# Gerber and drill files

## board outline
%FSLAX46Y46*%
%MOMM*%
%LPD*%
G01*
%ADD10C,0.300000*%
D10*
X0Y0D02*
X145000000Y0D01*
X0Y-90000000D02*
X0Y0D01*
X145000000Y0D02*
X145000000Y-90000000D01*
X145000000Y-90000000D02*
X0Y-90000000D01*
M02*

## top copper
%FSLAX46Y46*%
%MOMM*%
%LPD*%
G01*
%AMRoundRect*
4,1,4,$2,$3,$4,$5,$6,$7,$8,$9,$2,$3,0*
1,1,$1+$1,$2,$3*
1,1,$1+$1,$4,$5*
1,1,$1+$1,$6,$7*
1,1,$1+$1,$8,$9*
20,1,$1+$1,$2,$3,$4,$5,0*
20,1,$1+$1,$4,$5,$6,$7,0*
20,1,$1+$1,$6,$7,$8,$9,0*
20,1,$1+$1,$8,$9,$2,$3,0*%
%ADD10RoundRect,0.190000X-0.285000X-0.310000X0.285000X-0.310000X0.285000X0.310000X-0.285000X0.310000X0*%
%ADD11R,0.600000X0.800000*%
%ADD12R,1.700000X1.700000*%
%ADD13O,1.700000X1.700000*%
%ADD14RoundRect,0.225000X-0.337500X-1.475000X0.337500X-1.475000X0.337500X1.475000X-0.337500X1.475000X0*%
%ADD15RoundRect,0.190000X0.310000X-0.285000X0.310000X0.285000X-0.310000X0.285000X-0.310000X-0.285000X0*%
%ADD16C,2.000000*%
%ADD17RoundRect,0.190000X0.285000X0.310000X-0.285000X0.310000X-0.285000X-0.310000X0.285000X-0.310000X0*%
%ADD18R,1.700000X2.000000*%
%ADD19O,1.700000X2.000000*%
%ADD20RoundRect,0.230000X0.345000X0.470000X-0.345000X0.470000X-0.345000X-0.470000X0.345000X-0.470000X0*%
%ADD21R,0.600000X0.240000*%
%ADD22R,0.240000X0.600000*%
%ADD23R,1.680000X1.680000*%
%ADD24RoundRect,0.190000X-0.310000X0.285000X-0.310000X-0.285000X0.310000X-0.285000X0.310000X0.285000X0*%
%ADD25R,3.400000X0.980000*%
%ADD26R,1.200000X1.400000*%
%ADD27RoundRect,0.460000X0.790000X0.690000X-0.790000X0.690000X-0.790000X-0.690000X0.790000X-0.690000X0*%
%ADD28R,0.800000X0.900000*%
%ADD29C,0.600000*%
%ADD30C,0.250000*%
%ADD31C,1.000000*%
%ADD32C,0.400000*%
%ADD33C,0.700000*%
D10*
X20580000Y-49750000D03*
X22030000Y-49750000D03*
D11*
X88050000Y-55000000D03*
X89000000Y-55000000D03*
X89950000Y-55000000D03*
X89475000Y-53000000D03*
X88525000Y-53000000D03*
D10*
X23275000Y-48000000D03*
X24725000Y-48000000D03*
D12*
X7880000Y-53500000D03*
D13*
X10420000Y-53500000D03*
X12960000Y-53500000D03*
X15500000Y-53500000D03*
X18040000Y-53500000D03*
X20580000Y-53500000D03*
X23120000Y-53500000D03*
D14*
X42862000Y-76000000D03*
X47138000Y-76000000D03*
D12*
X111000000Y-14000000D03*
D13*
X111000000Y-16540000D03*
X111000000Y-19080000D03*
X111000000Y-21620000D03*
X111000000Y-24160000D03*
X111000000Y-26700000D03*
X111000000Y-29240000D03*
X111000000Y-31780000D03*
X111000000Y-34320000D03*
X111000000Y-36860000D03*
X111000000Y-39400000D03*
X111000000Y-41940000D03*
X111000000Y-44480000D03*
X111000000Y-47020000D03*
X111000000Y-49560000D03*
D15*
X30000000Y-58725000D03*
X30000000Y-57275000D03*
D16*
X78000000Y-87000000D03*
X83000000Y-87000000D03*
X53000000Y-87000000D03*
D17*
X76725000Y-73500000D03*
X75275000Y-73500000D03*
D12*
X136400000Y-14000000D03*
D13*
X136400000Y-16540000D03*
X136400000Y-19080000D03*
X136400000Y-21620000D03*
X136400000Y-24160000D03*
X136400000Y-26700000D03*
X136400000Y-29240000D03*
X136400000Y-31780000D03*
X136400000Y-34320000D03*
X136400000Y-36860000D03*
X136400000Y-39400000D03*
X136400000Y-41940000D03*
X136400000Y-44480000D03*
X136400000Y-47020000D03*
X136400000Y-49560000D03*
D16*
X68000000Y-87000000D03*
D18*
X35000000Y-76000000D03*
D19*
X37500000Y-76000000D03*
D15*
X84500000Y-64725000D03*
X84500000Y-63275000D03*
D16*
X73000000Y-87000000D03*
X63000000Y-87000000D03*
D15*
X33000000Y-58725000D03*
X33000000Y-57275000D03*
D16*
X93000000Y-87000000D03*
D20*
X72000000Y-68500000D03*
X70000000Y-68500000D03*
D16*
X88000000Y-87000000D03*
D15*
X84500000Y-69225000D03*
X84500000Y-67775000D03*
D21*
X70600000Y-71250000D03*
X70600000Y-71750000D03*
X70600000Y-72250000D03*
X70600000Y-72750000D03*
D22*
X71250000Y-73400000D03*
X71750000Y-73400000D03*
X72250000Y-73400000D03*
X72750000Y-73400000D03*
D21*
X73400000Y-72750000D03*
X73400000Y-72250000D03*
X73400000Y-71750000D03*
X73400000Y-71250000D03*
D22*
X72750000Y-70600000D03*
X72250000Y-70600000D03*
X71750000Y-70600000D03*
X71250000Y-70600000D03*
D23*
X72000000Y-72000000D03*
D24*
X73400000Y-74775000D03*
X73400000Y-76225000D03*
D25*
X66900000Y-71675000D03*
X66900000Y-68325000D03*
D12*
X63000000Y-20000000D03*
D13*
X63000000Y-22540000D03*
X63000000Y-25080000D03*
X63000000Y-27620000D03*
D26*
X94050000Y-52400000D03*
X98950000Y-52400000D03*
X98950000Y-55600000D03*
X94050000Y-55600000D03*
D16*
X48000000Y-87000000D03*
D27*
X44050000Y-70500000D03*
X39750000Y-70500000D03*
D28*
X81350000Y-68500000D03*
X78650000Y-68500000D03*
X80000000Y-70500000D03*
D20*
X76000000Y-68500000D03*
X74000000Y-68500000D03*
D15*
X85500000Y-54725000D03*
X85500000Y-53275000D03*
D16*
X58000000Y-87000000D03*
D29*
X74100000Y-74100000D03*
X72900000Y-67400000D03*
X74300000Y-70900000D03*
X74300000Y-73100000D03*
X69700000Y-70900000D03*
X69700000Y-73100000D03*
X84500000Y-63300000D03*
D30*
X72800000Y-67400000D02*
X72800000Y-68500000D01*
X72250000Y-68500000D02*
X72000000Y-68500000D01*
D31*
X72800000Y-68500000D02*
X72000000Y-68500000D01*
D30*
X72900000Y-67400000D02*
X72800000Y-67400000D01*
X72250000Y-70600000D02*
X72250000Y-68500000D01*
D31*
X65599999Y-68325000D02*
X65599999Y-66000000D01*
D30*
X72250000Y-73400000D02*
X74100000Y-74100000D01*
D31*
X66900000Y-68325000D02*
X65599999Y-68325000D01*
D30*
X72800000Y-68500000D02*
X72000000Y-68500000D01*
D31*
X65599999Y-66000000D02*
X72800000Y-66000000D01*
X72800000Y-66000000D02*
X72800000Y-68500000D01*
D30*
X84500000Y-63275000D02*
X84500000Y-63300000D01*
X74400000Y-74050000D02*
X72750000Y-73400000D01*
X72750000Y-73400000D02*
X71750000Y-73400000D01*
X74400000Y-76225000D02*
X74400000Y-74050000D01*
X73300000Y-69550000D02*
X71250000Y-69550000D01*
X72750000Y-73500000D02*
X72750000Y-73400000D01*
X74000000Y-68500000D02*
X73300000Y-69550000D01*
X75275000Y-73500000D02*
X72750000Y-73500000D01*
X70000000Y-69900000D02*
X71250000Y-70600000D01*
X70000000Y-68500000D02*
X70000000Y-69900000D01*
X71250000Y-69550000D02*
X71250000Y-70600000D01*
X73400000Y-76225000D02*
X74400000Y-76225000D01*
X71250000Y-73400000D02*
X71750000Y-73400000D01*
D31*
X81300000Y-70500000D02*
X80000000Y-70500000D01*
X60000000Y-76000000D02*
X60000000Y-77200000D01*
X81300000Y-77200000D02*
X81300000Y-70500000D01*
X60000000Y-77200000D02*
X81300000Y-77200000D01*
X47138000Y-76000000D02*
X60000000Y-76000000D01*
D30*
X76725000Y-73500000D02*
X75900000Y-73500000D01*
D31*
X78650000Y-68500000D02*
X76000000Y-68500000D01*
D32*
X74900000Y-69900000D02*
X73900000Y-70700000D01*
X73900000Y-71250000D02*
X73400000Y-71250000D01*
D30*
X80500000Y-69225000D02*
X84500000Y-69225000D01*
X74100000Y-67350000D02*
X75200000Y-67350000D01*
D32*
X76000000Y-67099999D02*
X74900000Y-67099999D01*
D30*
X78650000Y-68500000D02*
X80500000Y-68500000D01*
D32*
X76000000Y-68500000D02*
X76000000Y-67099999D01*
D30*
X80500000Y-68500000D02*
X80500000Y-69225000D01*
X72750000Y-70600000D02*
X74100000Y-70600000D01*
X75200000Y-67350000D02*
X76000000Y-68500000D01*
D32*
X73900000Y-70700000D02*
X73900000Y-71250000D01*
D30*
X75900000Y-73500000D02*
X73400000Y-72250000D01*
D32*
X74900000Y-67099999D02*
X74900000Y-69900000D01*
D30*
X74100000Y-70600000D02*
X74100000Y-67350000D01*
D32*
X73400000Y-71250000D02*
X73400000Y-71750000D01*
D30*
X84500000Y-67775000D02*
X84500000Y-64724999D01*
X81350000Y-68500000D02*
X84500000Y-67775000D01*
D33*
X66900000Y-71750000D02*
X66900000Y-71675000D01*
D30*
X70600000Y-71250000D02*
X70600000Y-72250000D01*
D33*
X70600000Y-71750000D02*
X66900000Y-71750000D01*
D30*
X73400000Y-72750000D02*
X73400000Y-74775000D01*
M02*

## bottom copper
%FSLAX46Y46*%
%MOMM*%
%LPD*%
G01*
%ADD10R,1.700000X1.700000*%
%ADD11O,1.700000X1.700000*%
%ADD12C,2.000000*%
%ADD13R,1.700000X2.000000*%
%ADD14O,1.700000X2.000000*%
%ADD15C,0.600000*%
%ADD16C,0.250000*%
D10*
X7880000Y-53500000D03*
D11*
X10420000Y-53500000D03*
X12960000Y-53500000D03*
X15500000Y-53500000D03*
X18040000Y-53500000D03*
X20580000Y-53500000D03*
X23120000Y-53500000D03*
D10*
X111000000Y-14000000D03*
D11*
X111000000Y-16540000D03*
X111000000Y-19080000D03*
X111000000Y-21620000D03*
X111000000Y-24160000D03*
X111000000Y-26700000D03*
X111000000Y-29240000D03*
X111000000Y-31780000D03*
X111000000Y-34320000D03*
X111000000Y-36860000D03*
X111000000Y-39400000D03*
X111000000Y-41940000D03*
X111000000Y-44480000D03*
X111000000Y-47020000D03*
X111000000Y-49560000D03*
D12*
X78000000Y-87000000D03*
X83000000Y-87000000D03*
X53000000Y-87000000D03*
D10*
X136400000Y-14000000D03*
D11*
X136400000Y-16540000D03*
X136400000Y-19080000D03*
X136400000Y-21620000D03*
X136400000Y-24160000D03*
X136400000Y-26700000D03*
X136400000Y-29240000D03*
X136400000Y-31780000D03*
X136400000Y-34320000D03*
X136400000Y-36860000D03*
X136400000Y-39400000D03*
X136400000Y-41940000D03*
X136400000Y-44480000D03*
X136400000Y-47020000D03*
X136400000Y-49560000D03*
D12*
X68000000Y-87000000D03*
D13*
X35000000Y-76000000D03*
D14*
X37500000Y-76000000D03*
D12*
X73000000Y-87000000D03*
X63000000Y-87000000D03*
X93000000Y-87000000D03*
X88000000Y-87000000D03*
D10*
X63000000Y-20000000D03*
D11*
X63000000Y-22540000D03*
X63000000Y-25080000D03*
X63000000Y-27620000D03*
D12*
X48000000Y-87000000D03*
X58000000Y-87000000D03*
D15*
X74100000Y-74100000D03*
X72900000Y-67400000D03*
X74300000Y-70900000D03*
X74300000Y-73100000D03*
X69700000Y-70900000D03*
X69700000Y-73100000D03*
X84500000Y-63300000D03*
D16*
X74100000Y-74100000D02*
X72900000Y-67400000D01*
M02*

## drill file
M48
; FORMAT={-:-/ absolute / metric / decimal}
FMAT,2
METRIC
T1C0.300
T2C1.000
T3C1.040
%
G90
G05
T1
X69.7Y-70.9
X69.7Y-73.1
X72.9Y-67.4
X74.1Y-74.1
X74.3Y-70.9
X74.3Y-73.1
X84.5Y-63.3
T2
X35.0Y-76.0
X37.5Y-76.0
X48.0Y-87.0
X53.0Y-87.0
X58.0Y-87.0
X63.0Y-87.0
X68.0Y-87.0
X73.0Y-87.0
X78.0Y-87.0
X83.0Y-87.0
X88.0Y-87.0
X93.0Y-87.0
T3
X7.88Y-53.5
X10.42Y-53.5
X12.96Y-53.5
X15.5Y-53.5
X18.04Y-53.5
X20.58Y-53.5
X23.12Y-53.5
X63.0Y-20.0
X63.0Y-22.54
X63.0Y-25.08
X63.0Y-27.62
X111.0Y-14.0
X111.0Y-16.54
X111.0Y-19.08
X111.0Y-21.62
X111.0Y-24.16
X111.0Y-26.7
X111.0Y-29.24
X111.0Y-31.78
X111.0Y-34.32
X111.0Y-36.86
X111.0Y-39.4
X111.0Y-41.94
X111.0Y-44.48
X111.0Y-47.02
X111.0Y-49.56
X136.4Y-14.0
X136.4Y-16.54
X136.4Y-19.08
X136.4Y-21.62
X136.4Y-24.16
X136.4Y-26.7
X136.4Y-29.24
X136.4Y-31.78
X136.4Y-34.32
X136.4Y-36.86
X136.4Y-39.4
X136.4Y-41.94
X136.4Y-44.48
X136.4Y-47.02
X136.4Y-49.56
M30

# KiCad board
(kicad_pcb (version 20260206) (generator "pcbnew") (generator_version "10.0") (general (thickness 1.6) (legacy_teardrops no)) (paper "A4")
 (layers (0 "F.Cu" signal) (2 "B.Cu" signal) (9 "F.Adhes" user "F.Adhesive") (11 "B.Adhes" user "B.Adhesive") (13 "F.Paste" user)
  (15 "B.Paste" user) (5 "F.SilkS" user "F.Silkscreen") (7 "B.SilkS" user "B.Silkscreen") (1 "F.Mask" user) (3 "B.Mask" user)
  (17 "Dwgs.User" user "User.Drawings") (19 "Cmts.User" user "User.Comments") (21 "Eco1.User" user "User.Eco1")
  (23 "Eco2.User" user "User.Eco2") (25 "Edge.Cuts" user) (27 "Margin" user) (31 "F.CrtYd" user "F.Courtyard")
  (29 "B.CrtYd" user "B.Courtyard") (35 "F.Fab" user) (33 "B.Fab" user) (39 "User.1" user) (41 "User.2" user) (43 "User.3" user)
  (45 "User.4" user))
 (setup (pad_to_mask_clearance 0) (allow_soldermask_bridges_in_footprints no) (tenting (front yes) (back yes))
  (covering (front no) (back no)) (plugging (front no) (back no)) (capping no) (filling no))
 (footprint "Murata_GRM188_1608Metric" (layer "F.Cu") (at 21.305 49.75)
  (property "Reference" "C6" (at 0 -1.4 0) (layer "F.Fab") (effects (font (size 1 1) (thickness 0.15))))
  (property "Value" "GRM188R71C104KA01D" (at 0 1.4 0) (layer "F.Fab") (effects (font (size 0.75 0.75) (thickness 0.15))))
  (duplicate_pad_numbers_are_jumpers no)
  (pad "1" smd roundrect (at -0.725 0) (size 0.95 1) (layers "F.Cu" "F.Mask" "F.Paste") (roundrect_rratio 0.2) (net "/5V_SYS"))
  (pad "2" smd roundrect (at 0.725 0) (size 0.95 1) (layers "F.Cu" "F.Mask" "F.Paste") (roundrect_rratio 0.2) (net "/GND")))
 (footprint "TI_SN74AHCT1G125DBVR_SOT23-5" (layer "F.Cu") (at 89 54)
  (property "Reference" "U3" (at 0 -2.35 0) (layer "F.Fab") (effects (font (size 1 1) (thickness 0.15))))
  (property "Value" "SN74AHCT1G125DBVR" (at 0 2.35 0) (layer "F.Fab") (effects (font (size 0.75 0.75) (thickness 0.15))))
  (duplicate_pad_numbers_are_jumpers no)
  (pad "1" smd rect (at -0.95 1) (size 0.6 0.8) (layers "F.Cu" "F.Mask" "F.Paste") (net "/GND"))
  (pad "2" smd rect (at 0 1) (size 0.6 0.8) (layers "F.Cu" "F.Mask" "F.Paste") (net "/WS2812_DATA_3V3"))
  (pad "3" smd rect (at 0.95 1) (size 0.6 0.8) (layers "F.Cu" "F.Mask" "F.Paste") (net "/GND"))
  (pad "4" smd rect (at 0.475 -1) (size 0.6 0.8) (layers "F.Cu" "F.Mask" "F.Paste") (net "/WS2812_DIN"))
  (pad "5" smd rect (at -0.475 -1) (size 0.6 0.8) (layers "F.Cu" "F.Mask" "F.Paste") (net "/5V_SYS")))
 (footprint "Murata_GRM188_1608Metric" (layer "F.Cu") (at 24 48)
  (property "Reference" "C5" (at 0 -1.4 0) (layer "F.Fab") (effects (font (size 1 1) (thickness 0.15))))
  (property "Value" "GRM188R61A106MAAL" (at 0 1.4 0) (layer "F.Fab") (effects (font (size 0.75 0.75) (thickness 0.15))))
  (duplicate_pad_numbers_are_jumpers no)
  (pad "1" smd roundrect (at -0.725 0) (size 0.95 1) (layers "F.Cu" "F.Mask" "F.Paste") (roundrect_rratio 0.2) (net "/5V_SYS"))
  (pad "2" smd roundrect (at 0.725 0) (size 0.95 1) (layers "F.Cu" "F.Mask" "F.Paste") (roundrect_rratio 0.2) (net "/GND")))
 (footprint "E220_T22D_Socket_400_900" (layer "F.Cu") (at 5 52)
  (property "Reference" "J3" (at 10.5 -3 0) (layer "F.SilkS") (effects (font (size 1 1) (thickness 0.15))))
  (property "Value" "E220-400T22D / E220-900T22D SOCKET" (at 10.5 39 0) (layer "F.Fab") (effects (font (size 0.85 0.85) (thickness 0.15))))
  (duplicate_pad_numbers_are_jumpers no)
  (pad "1" thru_hole rect (at 2.88 1.5) (size 1.7 1.7) (drill 1.04) (layers "*.Cu" "*.Mask") (remove_unused_layers no) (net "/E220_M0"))
  (pad "2" thru_hole oval (at 5.42 1.5) (size 1.7 1.7) (drill 1.04) (layers "*.Cu" "*.Mask") (remove_unused_layers no) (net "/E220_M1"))
  (pad "3" thru_hole oval (at 7.96 1.5) (size 1.7 1.7) (drill 1.04) (layers "*.Cu" "*.Mask") (remove_unused_layers no) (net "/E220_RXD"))
  (pad "4" thru_hole oval (at 10.5 1.5) (size 1.7 1.7) (drill 1.04) (layers "*.Cu" "*.Mask") (remove_unused_layers no) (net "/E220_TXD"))
  (pad "5" thru_hole oval (at 13.04 1.5) (size 1.7 1.7) (drill 1.04) (layers "*.Cu" "*.Mask") (remove_unused_layers no) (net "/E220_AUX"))
  (pad "6" thru_hole oval (at 15.58 1.5) (size 1.7 1.7) (drill 1.04) (layers "*.Cu" "*.Mask") (remove_unused_layers no) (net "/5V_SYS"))
  (pad "7" thru_hole oval (at 18.12 1.5) (size 1.7 1.7) (drill 1.04) (layers "*.Cu" "*.Mask") (remove_unused_layers no) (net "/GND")))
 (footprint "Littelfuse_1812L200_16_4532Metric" (layer "F.Cu") (at 45 76)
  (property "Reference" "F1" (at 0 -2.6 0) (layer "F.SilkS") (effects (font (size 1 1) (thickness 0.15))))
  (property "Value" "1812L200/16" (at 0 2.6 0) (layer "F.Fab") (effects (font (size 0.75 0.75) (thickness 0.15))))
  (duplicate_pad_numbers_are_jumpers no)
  (pad "1" smd roundrect (at -2.138 0) (size 1.125 3.4) (layers "F.Cu" "F.Mask" "F.Paste") (roundrect_rratio 0.2) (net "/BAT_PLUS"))
  (pad "2" smd roundrect (at 2.138 0) (size 1.125 3.4) (layers "F.Cu" "F.Mask" "F.Paste") (roundrect_rratio 0.2) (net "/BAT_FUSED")))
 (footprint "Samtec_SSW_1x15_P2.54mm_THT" (layer "F.Cu") (at 111 14)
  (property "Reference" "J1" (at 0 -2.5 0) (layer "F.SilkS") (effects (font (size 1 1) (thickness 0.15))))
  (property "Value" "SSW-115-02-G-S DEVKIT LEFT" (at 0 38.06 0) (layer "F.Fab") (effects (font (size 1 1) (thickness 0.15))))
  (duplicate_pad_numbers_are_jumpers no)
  (pad "1" thru_hole rect (at 0 0) (size 1.7 1.7) (drill 1.04) (layers "*.Cu" "*.Mask") (remove_unused_layers no) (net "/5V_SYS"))
  (pad "2" thru_hole oval (at 0 2.54) (size 1.7 1.7) (drill 1.04) (layers "*.Cu" "*.Mask") (remove_unused_layers no) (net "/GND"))
  (pad "3" thru_hole oval (at 0 5.08) (size 1.7 1.7) (drill 1.04) (layers "*.Cu" "*.Mask") (remove_unused_layers no))
  (pad "4" thru_hole oval (at 0 7.62) (size 1.7 1.7) (drill 1.04) (layers "*.Cu" "*.Mask") (remove_unused_layers no))
  (pad "5" thru_hole oval (at 0 10.16) (size 1.7 1.7) (drill 1.04) (layers "*.Cu" "*.Mask") (remove_unused_layers no))
  (pad "6" thru_hole oval (at 0 12.7) (size 1.7 1.7) (drill 1.04) (layers "*.Cu" "*.Mask") (remove_unused_layers no) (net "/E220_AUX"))
  (pad "7" thru_hole oval (at 0 15.24) (size 1.7 1.7) (drill 1.04) (layers "*.Cu" "*.Mask") (remove_unused_layers no) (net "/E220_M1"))
  (pad "8" thru_hole oval (at 0 17.78) (size 1.7 1.7) (drill 1.04) (layers "*.Cu" "*.Mask") (remove_unused_layers no) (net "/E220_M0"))
  (pad "9" thru_hole oval (at 0 20.32) (size 1.7 1.7) (drill 1.04) (layers "*.Cu" "*.Mask") (remove_unused_layers no))
  (pad "10" thru_hole oval (at 0 22.86) (size 1.7 1.7) (drill 1.04) (layers "*.Cu" "*.Mask") (remove_unused_layers no))
  (pad "11" thru_hole oval (at 0 25.4) (size 1.7 1.7) (drill 1.04) (layers "*.Cu" "*.Mask") (remove_unused_layers no))
  (pad "12" thru_hole oval (at 0 27.94) (size 1.7 1.7) (drill 1.04) (layers "*.Cu" "*.Mask") (remove_unused_layers no))
  (pad "13" thru_hole oval (at 0 30.48) (size 1.7 1.7) (drill 1.04) (layers "*.Cu" "*.Mask") (remove_unused_layers no))
  (pad "14" thru_hole oval (at 0 33.02) (size 1.7 1.7) (drill 1.04) (layers "*.Cu" "*.Mask") (remove_unused_layers no))
  (pad "15" thru_hole oval (at 0 35.56) (size 1.7 1.7) (drill 1.04) (layers "*.Cu" "*.Mask") (remove_unused_layers no)))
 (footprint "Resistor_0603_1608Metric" (layer "F.Cu") (at 30 58 90)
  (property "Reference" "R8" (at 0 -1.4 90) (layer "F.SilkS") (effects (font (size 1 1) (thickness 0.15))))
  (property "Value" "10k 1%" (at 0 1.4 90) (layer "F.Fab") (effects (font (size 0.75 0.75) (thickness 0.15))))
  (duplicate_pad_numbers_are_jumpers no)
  (pad "1" smd roundrect (at -0.725 0 90) (size 0.95 1) (layers "F.Cu" "F.Mask" "F.Paste") (roundrect_rratio 0.2) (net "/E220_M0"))
  (pad "2" smd roundrect (at 0.725 0 90) (size 0.95 1) (layers "F.Cu" "F.Mask" "F.Paste") (roundrect_rratio 0.2) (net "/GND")))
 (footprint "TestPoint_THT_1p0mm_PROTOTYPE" (layer "F.Cu") (at 78 87)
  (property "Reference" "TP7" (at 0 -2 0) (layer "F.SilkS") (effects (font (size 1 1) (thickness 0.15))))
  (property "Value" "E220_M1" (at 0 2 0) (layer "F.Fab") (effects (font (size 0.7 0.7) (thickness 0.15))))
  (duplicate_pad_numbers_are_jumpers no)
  (pad "1" thru_hole circle (at 0 0) (size 2 2) (drill 1) (layers "*.Cu" "*.Mask") (remove_unused_layers no) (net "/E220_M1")))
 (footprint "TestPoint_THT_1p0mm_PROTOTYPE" (layer "F.Cu") (at 83 87)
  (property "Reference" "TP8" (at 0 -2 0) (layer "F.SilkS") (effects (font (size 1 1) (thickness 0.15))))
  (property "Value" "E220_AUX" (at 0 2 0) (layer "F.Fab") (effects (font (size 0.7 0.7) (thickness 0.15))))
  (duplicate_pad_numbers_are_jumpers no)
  (pad "1" thru_hole circle (at 0 0) (size 2 2) (drill 1) (layers "*.Cu" "*.Mask") (remove_unused_layers no) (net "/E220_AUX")))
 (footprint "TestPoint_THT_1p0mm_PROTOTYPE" (layer "F.Cu") (at 53 87)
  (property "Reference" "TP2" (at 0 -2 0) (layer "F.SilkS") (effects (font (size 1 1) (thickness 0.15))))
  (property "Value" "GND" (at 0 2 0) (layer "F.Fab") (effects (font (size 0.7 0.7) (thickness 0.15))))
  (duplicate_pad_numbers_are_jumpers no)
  (pad "1" thru_hole circle (at 0 0) (size 2 2) (drill 1) (layers "*.Cu" "*.Mask") (remove_unused_layers no) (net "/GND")))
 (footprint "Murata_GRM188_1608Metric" (layer "F.Cu") (at 76 73.5 180)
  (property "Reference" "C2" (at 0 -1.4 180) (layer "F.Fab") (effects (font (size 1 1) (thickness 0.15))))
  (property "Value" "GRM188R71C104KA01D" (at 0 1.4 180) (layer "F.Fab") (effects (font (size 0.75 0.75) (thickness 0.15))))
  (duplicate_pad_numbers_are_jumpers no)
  (pad "1" smd roundrect (at -0.725 0 180) (size 0.95 1) (layers "F.Cu" "F.Mask" "F.Paste") (roundrect_rratio 0.2) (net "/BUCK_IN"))
  (pad "2" smd roundrect (at 0.725 0 180) (size 0.95 1) (layers "F.Cu" "F.Mask" "F.Paste") (roundrect_rratio 0.2) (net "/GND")))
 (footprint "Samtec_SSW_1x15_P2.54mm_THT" (layer "F.Cu") (at 136.4 14)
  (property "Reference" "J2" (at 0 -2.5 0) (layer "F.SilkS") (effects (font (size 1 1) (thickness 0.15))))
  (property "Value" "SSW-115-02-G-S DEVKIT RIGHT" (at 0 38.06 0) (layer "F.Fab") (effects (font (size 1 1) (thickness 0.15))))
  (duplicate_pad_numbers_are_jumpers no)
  (pad "1" thru_hole rect (at 0 0) (size 1.7 1.7) (drill 1.04) (layers "*.Cu" "*.Mask") (remove_unused_layers no) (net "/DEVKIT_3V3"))
  (pad "2" thru_hole oval (at 0 2.54) (size 1.7 1.7) (drill 1.04) (layers "*.Cu" "*.Mask") (remove_unused_layers no) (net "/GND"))
  (pad "3" thru_hole oval (at 0 5.08) (size 1.7 1.7) (drill 1.04) (layers "*.Cu" "*.Mask") (remove_unused_layers no))
  (pad "4" thru_hole oval (at 0 7.62) (size 1.7 1.7) (drill 1.04) (layers "*.Cu" "*.Mask") (remove_unused_layers no))
  (pad "5" thru_hole oval (at 0 10.16) (size 1.7 1.7) (drill 1.04) (layers "*.Cu" "*.Mask") (remove_unused_layers no)
   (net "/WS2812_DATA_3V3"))
  (pad "6" thru_hole oval (at 0 12.7) (size 1.7 1.7) (drill 1.04) (layers "*.Cu" "*.Mask") (remove_unused_layers no) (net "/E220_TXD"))
  (pad "7" thru_hole oval (at 0 15.24) (size 1.7 1.7) (drill 1.04) (layers "*.Cu" "*.Mask") (remove_unused_layers no) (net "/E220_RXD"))
  (pad "8" thru_hole oval (at 0 17.78) (size 1.7 1.7) (drill 1.04) (layers "*.Cu" "*.Mask") (remove_unused_layers no))
  (pad "9" thru_hole oval (at 0 20.32) (size 1.7 1.7) (drill 1.04) (layers "*.Cu" "*.Mask") (remove_unused_layers no))
  (pad "10" thru_hole oval (at 0 22.86) (size 1.7 1.7) (drill 1.04) (layers "*.Cu" "*.Mask") (remove_unused_layers no))
  (pad "11" thru_hole oval (at 0 25.4) (size 1.7 1.7) (drill 1.04) (layers "*.Cu" "*.Mask") (remove_unused_layers no) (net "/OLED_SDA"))
  (pad "12" thru_hole oval (at 0 27.94) (size 1.7 1.7) (drill 1.04) (layers "*.Cu" "*.Mask") (remove_unused_layers no))
  (pad "13" thru_hole oval (at 0 30.48) (size 1.7 1.7) (drill 1.04) (layers "*.Cu" "*.Mask") (remove_unused_layers no))
  (pad "14" thru_hole oval (at 0 33.02) (size 1.7 1.7) (drill 1.04) (layers "*.Cu" "*.Mask") (remove_unused_layers no) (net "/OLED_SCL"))
  (pad "15" thru_hole oval (at 0 35.56) (size 1.7 1.7) (drill 1.04) (layers "*.Cu" "*.Mask") (remove_unused_layers no)))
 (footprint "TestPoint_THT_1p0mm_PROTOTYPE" (layer "F.Cu") (at 68 87)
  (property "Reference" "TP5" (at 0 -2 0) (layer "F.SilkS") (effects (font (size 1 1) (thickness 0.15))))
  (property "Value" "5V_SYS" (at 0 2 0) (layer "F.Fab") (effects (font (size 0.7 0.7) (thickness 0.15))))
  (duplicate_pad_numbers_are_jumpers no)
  (pad "1" thru_hole circle (at 0 0) (size 2 2) (drill 1) (layers "*.Cu" "*.Mask") (remove_unused_layers no) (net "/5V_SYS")))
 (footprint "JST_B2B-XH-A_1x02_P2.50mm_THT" (layer "F.Cu") (at 35 76)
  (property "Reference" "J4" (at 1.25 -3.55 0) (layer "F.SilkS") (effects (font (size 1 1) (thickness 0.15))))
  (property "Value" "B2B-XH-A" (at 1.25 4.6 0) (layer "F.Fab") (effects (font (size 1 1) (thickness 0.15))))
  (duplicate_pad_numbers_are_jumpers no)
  (pad "1" thru_hole rect (at 0 0) (size 1.7 2) (drill 1) (layers "*.Cu" "*.Mask") (remove_unused_layers no) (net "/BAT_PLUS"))
  (pad "2" thru_hole oval (at 2.5 0) (size 1.7 2) (drill 1) (layers "*.Cu" "*.Mask") (remove_unused_layers no) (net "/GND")))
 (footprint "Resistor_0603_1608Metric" (layer "F.Cu") (at 84.5 64 90)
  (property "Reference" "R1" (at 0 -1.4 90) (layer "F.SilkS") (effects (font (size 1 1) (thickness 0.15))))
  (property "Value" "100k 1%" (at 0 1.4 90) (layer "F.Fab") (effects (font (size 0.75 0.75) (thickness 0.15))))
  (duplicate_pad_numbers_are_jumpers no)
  (pad "1" smd roundrect (at -0.725 0 90) (size 0.95 1) (layers "F.Cu" "F.Mask" "F.Paste") (roundrect_rratio 0.2) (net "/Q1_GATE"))
  (pad "2" smd roundrect (at 0.725 0 90) (size 0.95 1) (layers "F.Cu" "F.Mask" "F.Paste") (roundrect_rratio 0.2) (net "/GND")))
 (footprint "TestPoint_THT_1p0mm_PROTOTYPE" (layer "F.Cu") (at 73 87)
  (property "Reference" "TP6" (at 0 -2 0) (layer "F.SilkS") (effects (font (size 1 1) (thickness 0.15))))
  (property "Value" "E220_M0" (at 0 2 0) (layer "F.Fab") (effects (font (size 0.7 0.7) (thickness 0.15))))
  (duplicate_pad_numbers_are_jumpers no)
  (pad "1" thru_hole circle (at 0 0) (size 2 2) (drill 1) (layers "*.Cu" "*.Mask") (remove_unused_layers no) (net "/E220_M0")))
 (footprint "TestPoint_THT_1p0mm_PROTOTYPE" (layer "F.Cu") (at 63 87)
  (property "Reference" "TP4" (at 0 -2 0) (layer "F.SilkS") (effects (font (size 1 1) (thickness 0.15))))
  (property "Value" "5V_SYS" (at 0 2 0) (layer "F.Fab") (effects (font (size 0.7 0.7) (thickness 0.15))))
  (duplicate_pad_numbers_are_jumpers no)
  (pad "1" thru_hole circle (at 0 0) (size 2 2) (drill 1) (layers "*.Cu" "*.Mask") (remove_unused_layers no) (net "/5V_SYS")))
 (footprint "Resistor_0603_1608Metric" (layer "F.Cu") (at 33 58 90)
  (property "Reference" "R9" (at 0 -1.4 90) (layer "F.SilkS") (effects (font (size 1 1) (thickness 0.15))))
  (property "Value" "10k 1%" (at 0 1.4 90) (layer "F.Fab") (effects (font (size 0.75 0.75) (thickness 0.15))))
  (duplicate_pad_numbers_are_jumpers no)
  (pad "1" smd roundrect (at -0.725 0 90) (size 0.95 1) (layers "F.Cu" "F.Mask" "F.Paste") (roundrect_rratio 0.2) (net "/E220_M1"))
  (pad "2" smd roundrect (at 0.725 0 90) (size 0.95 1) (layers "F.Cu" "F.Mask" "F.Paste") (roundrect_rratio 0.2) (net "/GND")))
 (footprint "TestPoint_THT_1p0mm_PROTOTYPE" (layer "F.Cu") (at 93 87)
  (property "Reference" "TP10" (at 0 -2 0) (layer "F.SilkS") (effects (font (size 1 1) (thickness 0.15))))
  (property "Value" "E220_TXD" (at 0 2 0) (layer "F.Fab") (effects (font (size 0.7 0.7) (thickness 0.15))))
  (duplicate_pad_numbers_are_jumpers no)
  (pad "1" thru_hole circle (at 0 0) (size 2 2) (drill 1) (layers "*.Cu" "*.Mask") (remove_unused_layers no) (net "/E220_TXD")))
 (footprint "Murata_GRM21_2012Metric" (layer "F.Cu") (at 71 68.5 180)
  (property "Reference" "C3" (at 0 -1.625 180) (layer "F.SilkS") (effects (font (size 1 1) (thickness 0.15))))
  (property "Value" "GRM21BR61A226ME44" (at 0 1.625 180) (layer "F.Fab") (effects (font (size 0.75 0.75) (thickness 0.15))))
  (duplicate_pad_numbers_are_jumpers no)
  (pad "1" smd roundrect (at -1 0 180) (size 1.15 1.4) (layers "F.Cu" "F.Mask" "F.Paste") (roundrect_rratio 0.2) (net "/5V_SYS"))
  (pad "2" smd roundrect (at 1 0 180) (size 1.15 1.4) (layers "F.Cu" "F.Mask" "F.Paste") (roundrect_rratio 0.2) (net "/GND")))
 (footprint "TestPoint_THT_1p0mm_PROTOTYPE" (layer "F.Cu") (at 88 87)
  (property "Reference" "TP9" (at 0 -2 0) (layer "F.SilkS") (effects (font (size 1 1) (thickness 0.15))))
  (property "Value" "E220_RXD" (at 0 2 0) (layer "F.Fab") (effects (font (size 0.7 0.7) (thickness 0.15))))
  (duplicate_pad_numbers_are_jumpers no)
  (pad "1" thru_hole circle (at 0 0) (size 2 2) (drill 1) (layers "*.Cu" "*.Mask") (remove_unused_layers no) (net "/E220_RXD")))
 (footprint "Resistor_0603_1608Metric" (layer "F.Cu") (at 84.5 68.5 90)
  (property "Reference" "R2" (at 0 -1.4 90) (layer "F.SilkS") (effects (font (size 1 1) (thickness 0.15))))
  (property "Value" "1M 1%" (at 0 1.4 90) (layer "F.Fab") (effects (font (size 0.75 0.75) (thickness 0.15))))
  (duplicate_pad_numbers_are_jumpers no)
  (pad "1" smd roundrect (at -0.725 0 90) (size 0.95 1) (layers "F.Cu" "F.Mask" "F.Paste") (roundrect_rratio 0.2) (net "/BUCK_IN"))
  (pad "2" smd roundrect (at 0.725 0 90) (size 0.95 1) (layers "F.Cu" "F.Mask" "F.Paste") (roundrect_rratio 0.2) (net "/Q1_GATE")))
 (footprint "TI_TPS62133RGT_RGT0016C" (layer "F.Cu") (at 72 72)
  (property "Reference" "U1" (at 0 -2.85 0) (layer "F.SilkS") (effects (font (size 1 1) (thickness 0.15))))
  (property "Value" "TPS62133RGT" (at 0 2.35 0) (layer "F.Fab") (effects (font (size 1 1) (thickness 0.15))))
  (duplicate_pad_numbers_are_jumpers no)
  (pad "" smd rect (at 0 0) (size 1.55 1.55) (layers "F.Paste"))
  (pad "1" smd rect (at -1.4 -0.75) (size 0.6 0.24) (layers "F.Cu" "F.Mask" "F.Paste") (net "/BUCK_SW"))
  (pad "2" smd rect (at -1.4 -0.25) (size 0.6 0.24) (layers "F.Cu" "F.Mask" "F.Paste") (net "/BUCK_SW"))
  (pad "3" smd rect (at -1.4 0.25) (size 0.6 0.24) (layers "F.Cu" "F.Mask" "F.Paste") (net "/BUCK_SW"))
  (pad "4" smd rect (at -1.4 0.75) (size 0.6 0.24) (layers "F.Cu" "F.Mask" "F.Paste"))
  (pad "5" smd rect (at -0.75 1.4) (size 0.24 0.6) (layers "F.Cu" "F.Mask" "F.Paste") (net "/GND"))
  (pad "6" smd rect (at -0.25 1.4) (size 0.24 0.6) (layers "F.Cu" "F.Mask" "F.Paste") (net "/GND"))
  (pad "7" smd rect (at 0.25 1.4) (size 0.24 0.6) (layers "F.Cu" "F.Mask" "F.Paste") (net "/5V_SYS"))
  (pad "8" smd rect (at 0.75 1.4) (size 0.24 0.6) (layers "F.Cu" "F.Mask" "F.Paste") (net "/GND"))
  (pad "9" smd rect (at 1.4 0.75) (size 0.6 0.24) (layers "F.Cu" "F.Mask" "F.Paste") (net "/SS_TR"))
  (pad "10" smd rect (at 1.4 0.25) (size 0.6 0.24) (layers "F.Cu" "F.Mask" "F.Paste") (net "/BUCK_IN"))
  (pad "11" smd rect (at 1.4 -0.25) (size 0.6 0.24) (layers "F.Cu" "F.Mask" "F.Paste") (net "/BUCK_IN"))
  (pad "12" smd rect (at 1.4 -0.75) (size 0.6 0.24) (layers "F.Cu" "F.Mask" "F.Paste") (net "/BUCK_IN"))
  (pad "13" smd rect (at 0.75 -1.4) (size 0.24 0.6) (layers "F.Cu" "F.Mask" "F.Paste") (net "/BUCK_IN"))
  (pad "14" smd rect (at 0.25 -1.4) (size 0.24 0.6) (layers "F.Cu" "F.Mask" "F.Paste") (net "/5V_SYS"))
  (pad "15" smd rect (at -0.25 -1.4) (size 0.24 0.6) (layers "F.Cu" "F.Mask" "F.Paste") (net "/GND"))
  (pad "16" smd rect (at -0.75 -1.4) (size 0.24 0.6) (layers "F.Cu" "F.Mask" "F.Paste") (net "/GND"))
  (pad "EP" smd rect (at 0 0) (size 1.68 1.68) (layers "F.Cu" "F.Mask") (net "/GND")))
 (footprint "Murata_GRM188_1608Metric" (layer "F.Cu") (at 73.4 75.5 -90)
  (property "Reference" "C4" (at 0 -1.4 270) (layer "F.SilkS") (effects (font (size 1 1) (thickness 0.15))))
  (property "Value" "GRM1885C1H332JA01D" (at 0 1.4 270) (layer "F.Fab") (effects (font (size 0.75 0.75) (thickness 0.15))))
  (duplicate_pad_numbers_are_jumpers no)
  (pad "1" smd roundrect (at -0.725 0 270) (size 0.95 1) (layers "F.Cu" "F.Mask" "F.Paste") (roundrect_rratio 0.2) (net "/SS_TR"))
  (pad "2" smd roundrect (at 0.725 0 270) (size 0.95 1) (layers "F.Cu" "F.Mask" "F.Paste") (roundrect_rratio 0.2) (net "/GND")))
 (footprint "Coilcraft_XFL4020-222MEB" (layer "F.Cu") (at 66.9 70 90)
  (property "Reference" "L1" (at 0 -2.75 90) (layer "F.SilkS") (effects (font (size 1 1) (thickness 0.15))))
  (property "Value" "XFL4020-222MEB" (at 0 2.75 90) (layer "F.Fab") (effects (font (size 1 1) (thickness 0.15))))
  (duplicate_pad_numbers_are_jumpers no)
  (pad "1" smd rect (at -1.675 0 90) (size 0.98 3.4) (layers "F.Cu" "F.Mask" "F.Paste") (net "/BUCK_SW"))
  (pad "2" smd rect (at 1.675 0 90) (size 0.98 3.4) (layers "F.Cu" "F.Mask" "F.Paste") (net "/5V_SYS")))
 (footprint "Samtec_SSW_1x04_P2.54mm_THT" (layer "F.Cu") (at 63 20)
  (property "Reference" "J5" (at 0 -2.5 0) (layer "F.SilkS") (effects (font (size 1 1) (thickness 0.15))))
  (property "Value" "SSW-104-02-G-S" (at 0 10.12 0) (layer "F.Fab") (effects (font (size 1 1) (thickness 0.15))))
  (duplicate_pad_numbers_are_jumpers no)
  (pad "1" thru_hole rect (at 0 0) (size 1.7 1.7) (drill 1.04) (layers "*.Cu" "*.Mask") (remove_unused_layers no) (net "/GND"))
  (pad "2" thru_hole oval (at 0 2.54) (size 1.7 1.7) (drill 1.04) (layers "*.Cu" "*.Mask") (remove_unused_layers no) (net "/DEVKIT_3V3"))
  (pad "3" thru_hole oval (at 0 5.08) (size 1.7 1.7) (drill 1.04) (layers "*.Cu" "*.Mask") (remove_unused_layers no) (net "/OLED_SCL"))
  (pad "4" thru_hole oval (at 0 7.62) (size 1.7 1.7) (drill 1.04) (layers "*.Cu" "*.Mask") (remove_unused_layers no) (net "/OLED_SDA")))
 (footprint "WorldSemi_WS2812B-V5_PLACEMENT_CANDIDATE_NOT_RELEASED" (layer "F.Cu") (at 96.5 54)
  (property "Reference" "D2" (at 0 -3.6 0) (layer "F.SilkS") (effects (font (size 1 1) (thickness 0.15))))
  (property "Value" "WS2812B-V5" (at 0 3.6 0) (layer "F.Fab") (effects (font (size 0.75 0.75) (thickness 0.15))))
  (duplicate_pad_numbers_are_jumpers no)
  (pad "1" smd rect (at -2.45 -1.6) (size 1.2 1.4) (layers "F.Cu" "F.Mask" "F.Paste") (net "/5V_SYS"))
  (pad "2" smd rect (at 2.45 -1.6) (size 1.2 1.4) (layers "F.Cu" "F.Mask" "F.Paste"))
  (pad "3" smd rect (at 2.45 1.6) (size 1.2 1.4) (layers "F.Cu" "F.Mask" "F.Paste") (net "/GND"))
  (pad "4" smd rect (at -2.45 1.6) (size 1.2 1.4) (layers "F.Cu" "F.Mask" "F.Paste") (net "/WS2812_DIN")))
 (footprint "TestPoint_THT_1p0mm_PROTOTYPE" (layer "F.Cu") (at 48 87)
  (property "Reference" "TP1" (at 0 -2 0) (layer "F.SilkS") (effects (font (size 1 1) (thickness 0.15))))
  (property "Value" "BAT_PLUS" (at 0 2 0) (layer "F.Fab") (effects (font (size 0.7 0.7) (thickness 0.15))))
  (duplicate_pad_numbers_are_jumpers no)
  (pad "1" thru_hole circle (at 0 0) (size 2 2) (drill 1) (layers "*.Cu" "*.Mask") (remove_unused_layers no) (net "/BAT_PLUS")))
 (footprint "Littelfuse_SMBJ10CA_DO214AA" (layer "F.Cu") (at 41.9 70.5 180)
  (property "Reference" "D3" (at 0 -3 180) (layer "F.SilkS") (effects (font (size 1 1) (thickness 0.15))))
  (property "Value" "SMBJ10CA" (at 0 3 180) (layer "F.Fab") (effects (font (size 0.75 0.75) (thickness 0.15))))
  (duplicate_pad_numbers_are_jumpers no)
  (pad "1" smd roundrect (at -2.15 0 180) (size 2.5 2.3) (layers "F.Cu" "F.Mask" "F.Paste") (roundrect_rratio 0.2) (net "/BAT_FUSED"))
  (pad "2" smd roundrect (at 2.15 0 180) (size 2.5 2.3) (layers "F.Cu" "F.Mask" "F.Paste") (roundrect_rratio 0.2) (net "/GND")))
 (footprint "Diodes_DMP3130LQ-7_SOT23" (layer "F.Cu") (at 80 69.5 180)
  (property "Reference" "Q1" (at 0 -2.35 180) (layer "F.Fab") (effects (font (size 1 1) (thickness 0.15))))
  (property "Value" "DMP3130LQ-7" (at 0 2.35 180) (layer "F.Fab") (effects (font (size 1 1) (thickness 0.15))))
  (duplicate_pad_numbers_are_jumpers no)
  (pad "1" smd rect (at -1.35 1 180) (size 0.8 0.9) (layers "F.Cu" "F.Mask" "F.Paste") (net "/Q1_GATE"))
  (pad "2" smd rect (at 1.35 1 180) (size 0.8 0.9) (layers "F.Cu" "F.Mask" "F.Paste") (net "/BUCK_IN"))
  (pad "3" smd rect (at 0 -1 180) (size 0.8 0.9) (layers "F.Cu" "F.Mask" "F.Paste") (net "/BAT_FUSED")))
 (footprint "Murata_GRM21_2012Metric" (layer "F.Cu") (at 75 68.5 180)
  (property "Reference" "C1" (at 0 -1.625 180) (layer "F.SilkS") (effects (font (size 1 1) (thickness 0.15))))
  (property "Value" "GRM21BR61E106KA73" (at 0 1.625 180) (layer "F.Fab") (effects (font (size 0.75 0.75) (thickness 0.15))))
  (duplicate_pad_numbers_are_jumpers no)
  (pad "1" smd roundrect (at -1 0 180) (size 1.15 1.4) (layers "F.Cu" "F.Mask" "F.Paste") (roundrect_rratio 0.2) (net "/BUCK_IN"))
  (pad "2" smd roundrect (at 1 0 180) (size 1.15 1.4) (layers "F.Cu" "F.Mask" "F.Paste") (roundrect_rratio 0.2) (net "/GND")))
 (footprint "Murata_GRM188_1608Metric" (layer "F.Cu") (at 85.5 54 90)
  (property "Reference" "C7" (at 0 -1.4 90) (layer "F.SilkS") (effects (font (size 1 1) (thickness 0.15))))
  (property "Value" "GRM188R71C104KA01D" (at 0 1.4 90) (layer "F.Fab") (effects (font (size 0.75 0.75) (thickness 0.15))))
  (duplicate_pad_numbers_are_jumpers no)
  (pad "1" smd roundrect (at -0.725 0 90) (size 0.95 1) (layers "F.Cu" "F.Mask" "F.Paste") (roundrect_rratio 0.2) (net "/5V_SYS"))
  (pad "2" smd roundrect (at 0.725 0 90) (size 0.95 1) (layers "F.Cu" "F.Mask" "F.Paste") (roundrect_rratio 0.2) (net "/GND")))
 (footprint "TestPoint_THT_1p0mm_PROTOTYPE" (layer "F.Cu") (at 58 87)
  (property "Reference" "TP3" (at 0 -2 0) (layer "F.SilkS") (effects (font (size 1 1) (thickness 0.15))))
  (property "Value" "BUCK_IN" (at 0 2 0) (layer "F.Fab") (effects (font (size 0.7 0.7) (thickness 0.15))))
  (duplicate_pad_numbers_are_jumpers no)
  (pad "1" thru_hole circle (at 0 0) (size 2 2) (drill 1) (layers "*.Cu" "*.Mask") (remove_unused_layers no) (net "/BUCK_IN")))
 (gr_line (start 0 0) (end 145 0) (stroke (width 0.3) (type default)) (layer "Edge.Cuts"))
 (gr_line (start 0 90) (end 0 0) (stroke (width 0.3) (type default)) (layer "Edge.Cuts"))
 (gr_line (start 145 0) (end 145 90) (stroke (width 0.3) (type default)) (layer "Edge.Cuts"))
 (gr_line (start 145 90) (end 0 90) (stroke (width 0.3) (type default)) (layer "Edge.Cuts"))
 (segment (start 72.8 67.4) (end 72.8 68.5) (width 0.25) (layer "F.Cu") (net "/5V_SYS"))
 (segment (start 72.25 68.5) (end 72 68.5) (width 0.25) (layer "F.Cu") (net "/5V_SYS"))
 (segment (start 72.8 68.5) (end 72 68.5) (width 1) (layer "F.Cu") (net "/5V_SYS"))
 (segment (start 72.9 67.4) (end 72.8 67.4) (width 0.25) (layer "F.Cu") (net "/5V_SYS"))
 (segment (start 72.25 70.6) (end 72.25 68.5) (width 0.25) (layer "F.Cu") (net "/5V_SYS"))
 (segment (start 65.599999 68.325) (end 65.599999 66) (width 1) (layer "F.Cu") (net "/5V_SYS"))
 (segment (start 72.25 73.4) (end 74.1 74.1) (width 0.25) (layer "F.Cu") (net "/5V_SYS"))
 (segment (start 66.9 68.325) (end 65.599999 68.325) (width 1) (layer "F.Cu") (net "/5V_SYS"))
 (segment (start 72.8 68.5) (end 72 68.5) (width 0.25) (layer "F.Cu") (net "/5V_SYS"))
 (segment (start 65.599999 66) (end 72.8 66) (width 1) (layer "F.Cu") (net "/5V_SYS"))
 (segment (start 72.8 66) (end 72.8 68.5) (width 1) (layer "F.Cu") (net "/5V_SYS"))
 (via (at 74.1 74.1) (size 0.6) (drill 0.3) (layers "F.Cu" "B.Cu") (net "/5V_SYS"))
 (via (at 72.9 67.4) (size 0.6) (drill 0.3) (layers "F.Cu" "B.Cu") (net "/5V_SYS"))
 (segment (start 74.1 74.1) (end 72.9 67.4) (width 0.25) (layer "B.Cu") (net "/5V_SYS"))
 (segment (start 84.5 63.275) (end 84.5 63.3) (width 0.25) (layer "F.Cu") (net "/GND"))
 (segment (start 74.4 74.05) (end 72.75 73.4) (width 0.25) (layer "F.Cu") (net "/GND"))
 (segment (start 72.75 73.4) (end 71.75 73.4) (width 0.25) (layer "F.Cu") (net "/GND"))
 (segment (start 74.4 76.225) (end 74.4 74.05) (width 0.25) (layer "F.Cu") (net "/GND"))
 (segment (start 73.3 69.55) (end 71.25 69.55) (width 0.25) (layer "F.Cu") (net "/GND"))
 (segment (start 72.75 73.5) (end 72.75 73.4) (width 0.25) (layer "F.Cu") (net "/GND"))
 (segment (start 74 68.5) (end 73.3 69.55) (width 0.25) (layer "F.Cu") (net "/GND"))
 (segment (start 75.275 73.5) (end 72.75 73.5) (width 0.25) (layer "F.Cu") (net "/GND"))
 (segment (start 70 69.9) (end 71.25 70.6) (width 0.25) (layer "F.Cu") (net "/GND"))
 (segment (start 70 68.5) (end 70 69.9) (width 0.25) (layer "F.Cu") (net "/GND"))
 (segment (start 71.25 69.55) (end 71.25 70.6) (width 0.25) (layer "F.Cu") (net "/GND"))
 (segment (start 73.4 76.225) (end 74.4 76.225) (width 0.25) (layer "F.Cu") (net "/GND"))
 (segment (start 71.25 73.4) (end 71.75 73.4) (width 0.25) (layer "F.Cu") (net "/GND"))
 (via (at 74.3 70.9) (size 0.6) (drill 0.3) (layers "F.Cu" "B.Cu") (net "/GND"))
 (via (at 74.3 73.1) (size 0.6) (drill 0.3) (layers "F.Cu" "B.Cu") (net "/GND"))
 (via (at 69.7 70.9) (size 0.6) (drill 0.3) (layers "F.Cu" "B.Cu") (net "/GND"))
 (via (at 69.7 73.1) (size 0.6) (drill 0.3) (layers "F.Cu" "B.Cu") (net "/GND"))
 (via (at 84.5 63.3) (size 0.6) (drill 0.3) (layers "F.Cu" "B.Cu") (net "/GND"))
 (segment (start 81.3 70.5) (end 80 70.5) (width 1) (layer "F.Cu") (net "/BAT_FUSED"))
 (segment (start 60 76) (end 60 77.2) (width 1) (layer "F.Cu") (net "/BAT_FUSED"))
 (segment (start 81.3 77.2) (end 81.3 70.5) (width 1) (layer "F.Cu") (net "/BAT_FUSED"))
 (segment (start 60 77.2) (end 81.3 77.2) (width 1) (layer "F.Cu") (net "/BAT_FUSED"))
 (segment (start 47.138 76) (end 60 76) (width 1) (layer "F.Cu") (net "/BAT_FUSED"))
 (segment (start 76.725 73.5) (end 75.9 73.5) (width 0.25) (layer "F.Cu") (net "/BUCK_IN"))
 (segment (start 78.65 68.5) (end 76 68.5) (width 1) (layer "F.Cu") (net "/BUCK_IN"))
 (segment (start 74.9 69.9) (end 73.9 70.7) (width 0.4) (layer "F.Cu") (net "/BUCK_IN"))
 (segment (start 73.9 71.25) (end 73.4 71.25) (width 0.4) (layer "F.Cu") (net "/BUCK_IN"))
 (segment (start 80.5 69.225) (end 84.5 69.225) (width 0.25) (layer "F.Cu") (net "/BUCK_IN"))
 (segment (start 74.1 67.35) (end 75.2 67.35) (width 0.25) (layer "F.Cu") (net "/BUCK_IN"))
 (segment (start 76 67.099999) (end 74.9 67.099999) (width 0.4) (layer "F.Cu") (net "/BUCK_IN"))
 (segment (start 78.65 68.5) (end 80.5 68.5) (width 0.25) (layer "F.Cu") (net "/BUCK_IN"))
 (segment (start 76 68.5) (end 76 67.099999) (width 0.4) (layer "F.Cu") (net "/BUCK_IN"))
 (segment (start 80.5 68.5) (end 80.5 69.225) (width 0.25) (layer "F.Cu") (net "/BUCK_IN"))
 (segment (start 72.75 70.6) (end 74.1 70.6) (width 0.25) (layer "F.Cu") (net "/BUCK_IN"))
 (segment (start 75.2 67.35) (end 76 68.5) (width 0.25) (layer "F.Cu") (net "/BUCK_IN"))
 (segment (start 73.9 70.7) (end 73.9 71.25) (width 0.4) (layer "F.Cu") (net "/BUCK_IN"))
 (segment (start 75.9 73.5) (end 73.4 72.25) (width 0.25) (layer "F.Cu") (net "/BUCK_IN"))
 (segment (start 74.9 67.099999) (end 74.9 69.9) (width 0.4) (layer "F.Cu") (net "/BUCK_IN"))
 (segment (start 74.1 70.6) (end 74.1 67.35) (width 0.25) (layer "F.Cu") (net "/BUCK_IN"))
 (segment (start 73.4 71.25) (end 73.4 71.75) (width 0.4) (layer "F.Cu") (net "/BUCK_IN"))
 (segment (start 84.5 67.775) (end 84.5 64.724999) (width 0.25) (layer "F.Cu") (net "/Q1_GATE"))
 (segment (start 81.35 68.5) (end 84.5 67.775) (width 0.25) (layer "F.Cu") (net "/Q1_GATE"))
 (segment (start 66.9 71.75) (end 66.9 71.675) (width 0.7) (layer "F.Cu") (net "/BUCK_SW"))
 (segment (start 70.6 71.25) (end 70.6 72.25) (width 0.25) (layer "F.Cu") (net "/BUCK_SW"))
 (segment (start 70.6 71.75) (end 66.9 71.75) (width 0.7) (layer "F.Cu") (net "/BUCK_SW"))
 (segment (start 73.4 72.75) (end 73.4 74.775) (width 0.25) (layer "F.Cu") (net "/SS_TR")))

